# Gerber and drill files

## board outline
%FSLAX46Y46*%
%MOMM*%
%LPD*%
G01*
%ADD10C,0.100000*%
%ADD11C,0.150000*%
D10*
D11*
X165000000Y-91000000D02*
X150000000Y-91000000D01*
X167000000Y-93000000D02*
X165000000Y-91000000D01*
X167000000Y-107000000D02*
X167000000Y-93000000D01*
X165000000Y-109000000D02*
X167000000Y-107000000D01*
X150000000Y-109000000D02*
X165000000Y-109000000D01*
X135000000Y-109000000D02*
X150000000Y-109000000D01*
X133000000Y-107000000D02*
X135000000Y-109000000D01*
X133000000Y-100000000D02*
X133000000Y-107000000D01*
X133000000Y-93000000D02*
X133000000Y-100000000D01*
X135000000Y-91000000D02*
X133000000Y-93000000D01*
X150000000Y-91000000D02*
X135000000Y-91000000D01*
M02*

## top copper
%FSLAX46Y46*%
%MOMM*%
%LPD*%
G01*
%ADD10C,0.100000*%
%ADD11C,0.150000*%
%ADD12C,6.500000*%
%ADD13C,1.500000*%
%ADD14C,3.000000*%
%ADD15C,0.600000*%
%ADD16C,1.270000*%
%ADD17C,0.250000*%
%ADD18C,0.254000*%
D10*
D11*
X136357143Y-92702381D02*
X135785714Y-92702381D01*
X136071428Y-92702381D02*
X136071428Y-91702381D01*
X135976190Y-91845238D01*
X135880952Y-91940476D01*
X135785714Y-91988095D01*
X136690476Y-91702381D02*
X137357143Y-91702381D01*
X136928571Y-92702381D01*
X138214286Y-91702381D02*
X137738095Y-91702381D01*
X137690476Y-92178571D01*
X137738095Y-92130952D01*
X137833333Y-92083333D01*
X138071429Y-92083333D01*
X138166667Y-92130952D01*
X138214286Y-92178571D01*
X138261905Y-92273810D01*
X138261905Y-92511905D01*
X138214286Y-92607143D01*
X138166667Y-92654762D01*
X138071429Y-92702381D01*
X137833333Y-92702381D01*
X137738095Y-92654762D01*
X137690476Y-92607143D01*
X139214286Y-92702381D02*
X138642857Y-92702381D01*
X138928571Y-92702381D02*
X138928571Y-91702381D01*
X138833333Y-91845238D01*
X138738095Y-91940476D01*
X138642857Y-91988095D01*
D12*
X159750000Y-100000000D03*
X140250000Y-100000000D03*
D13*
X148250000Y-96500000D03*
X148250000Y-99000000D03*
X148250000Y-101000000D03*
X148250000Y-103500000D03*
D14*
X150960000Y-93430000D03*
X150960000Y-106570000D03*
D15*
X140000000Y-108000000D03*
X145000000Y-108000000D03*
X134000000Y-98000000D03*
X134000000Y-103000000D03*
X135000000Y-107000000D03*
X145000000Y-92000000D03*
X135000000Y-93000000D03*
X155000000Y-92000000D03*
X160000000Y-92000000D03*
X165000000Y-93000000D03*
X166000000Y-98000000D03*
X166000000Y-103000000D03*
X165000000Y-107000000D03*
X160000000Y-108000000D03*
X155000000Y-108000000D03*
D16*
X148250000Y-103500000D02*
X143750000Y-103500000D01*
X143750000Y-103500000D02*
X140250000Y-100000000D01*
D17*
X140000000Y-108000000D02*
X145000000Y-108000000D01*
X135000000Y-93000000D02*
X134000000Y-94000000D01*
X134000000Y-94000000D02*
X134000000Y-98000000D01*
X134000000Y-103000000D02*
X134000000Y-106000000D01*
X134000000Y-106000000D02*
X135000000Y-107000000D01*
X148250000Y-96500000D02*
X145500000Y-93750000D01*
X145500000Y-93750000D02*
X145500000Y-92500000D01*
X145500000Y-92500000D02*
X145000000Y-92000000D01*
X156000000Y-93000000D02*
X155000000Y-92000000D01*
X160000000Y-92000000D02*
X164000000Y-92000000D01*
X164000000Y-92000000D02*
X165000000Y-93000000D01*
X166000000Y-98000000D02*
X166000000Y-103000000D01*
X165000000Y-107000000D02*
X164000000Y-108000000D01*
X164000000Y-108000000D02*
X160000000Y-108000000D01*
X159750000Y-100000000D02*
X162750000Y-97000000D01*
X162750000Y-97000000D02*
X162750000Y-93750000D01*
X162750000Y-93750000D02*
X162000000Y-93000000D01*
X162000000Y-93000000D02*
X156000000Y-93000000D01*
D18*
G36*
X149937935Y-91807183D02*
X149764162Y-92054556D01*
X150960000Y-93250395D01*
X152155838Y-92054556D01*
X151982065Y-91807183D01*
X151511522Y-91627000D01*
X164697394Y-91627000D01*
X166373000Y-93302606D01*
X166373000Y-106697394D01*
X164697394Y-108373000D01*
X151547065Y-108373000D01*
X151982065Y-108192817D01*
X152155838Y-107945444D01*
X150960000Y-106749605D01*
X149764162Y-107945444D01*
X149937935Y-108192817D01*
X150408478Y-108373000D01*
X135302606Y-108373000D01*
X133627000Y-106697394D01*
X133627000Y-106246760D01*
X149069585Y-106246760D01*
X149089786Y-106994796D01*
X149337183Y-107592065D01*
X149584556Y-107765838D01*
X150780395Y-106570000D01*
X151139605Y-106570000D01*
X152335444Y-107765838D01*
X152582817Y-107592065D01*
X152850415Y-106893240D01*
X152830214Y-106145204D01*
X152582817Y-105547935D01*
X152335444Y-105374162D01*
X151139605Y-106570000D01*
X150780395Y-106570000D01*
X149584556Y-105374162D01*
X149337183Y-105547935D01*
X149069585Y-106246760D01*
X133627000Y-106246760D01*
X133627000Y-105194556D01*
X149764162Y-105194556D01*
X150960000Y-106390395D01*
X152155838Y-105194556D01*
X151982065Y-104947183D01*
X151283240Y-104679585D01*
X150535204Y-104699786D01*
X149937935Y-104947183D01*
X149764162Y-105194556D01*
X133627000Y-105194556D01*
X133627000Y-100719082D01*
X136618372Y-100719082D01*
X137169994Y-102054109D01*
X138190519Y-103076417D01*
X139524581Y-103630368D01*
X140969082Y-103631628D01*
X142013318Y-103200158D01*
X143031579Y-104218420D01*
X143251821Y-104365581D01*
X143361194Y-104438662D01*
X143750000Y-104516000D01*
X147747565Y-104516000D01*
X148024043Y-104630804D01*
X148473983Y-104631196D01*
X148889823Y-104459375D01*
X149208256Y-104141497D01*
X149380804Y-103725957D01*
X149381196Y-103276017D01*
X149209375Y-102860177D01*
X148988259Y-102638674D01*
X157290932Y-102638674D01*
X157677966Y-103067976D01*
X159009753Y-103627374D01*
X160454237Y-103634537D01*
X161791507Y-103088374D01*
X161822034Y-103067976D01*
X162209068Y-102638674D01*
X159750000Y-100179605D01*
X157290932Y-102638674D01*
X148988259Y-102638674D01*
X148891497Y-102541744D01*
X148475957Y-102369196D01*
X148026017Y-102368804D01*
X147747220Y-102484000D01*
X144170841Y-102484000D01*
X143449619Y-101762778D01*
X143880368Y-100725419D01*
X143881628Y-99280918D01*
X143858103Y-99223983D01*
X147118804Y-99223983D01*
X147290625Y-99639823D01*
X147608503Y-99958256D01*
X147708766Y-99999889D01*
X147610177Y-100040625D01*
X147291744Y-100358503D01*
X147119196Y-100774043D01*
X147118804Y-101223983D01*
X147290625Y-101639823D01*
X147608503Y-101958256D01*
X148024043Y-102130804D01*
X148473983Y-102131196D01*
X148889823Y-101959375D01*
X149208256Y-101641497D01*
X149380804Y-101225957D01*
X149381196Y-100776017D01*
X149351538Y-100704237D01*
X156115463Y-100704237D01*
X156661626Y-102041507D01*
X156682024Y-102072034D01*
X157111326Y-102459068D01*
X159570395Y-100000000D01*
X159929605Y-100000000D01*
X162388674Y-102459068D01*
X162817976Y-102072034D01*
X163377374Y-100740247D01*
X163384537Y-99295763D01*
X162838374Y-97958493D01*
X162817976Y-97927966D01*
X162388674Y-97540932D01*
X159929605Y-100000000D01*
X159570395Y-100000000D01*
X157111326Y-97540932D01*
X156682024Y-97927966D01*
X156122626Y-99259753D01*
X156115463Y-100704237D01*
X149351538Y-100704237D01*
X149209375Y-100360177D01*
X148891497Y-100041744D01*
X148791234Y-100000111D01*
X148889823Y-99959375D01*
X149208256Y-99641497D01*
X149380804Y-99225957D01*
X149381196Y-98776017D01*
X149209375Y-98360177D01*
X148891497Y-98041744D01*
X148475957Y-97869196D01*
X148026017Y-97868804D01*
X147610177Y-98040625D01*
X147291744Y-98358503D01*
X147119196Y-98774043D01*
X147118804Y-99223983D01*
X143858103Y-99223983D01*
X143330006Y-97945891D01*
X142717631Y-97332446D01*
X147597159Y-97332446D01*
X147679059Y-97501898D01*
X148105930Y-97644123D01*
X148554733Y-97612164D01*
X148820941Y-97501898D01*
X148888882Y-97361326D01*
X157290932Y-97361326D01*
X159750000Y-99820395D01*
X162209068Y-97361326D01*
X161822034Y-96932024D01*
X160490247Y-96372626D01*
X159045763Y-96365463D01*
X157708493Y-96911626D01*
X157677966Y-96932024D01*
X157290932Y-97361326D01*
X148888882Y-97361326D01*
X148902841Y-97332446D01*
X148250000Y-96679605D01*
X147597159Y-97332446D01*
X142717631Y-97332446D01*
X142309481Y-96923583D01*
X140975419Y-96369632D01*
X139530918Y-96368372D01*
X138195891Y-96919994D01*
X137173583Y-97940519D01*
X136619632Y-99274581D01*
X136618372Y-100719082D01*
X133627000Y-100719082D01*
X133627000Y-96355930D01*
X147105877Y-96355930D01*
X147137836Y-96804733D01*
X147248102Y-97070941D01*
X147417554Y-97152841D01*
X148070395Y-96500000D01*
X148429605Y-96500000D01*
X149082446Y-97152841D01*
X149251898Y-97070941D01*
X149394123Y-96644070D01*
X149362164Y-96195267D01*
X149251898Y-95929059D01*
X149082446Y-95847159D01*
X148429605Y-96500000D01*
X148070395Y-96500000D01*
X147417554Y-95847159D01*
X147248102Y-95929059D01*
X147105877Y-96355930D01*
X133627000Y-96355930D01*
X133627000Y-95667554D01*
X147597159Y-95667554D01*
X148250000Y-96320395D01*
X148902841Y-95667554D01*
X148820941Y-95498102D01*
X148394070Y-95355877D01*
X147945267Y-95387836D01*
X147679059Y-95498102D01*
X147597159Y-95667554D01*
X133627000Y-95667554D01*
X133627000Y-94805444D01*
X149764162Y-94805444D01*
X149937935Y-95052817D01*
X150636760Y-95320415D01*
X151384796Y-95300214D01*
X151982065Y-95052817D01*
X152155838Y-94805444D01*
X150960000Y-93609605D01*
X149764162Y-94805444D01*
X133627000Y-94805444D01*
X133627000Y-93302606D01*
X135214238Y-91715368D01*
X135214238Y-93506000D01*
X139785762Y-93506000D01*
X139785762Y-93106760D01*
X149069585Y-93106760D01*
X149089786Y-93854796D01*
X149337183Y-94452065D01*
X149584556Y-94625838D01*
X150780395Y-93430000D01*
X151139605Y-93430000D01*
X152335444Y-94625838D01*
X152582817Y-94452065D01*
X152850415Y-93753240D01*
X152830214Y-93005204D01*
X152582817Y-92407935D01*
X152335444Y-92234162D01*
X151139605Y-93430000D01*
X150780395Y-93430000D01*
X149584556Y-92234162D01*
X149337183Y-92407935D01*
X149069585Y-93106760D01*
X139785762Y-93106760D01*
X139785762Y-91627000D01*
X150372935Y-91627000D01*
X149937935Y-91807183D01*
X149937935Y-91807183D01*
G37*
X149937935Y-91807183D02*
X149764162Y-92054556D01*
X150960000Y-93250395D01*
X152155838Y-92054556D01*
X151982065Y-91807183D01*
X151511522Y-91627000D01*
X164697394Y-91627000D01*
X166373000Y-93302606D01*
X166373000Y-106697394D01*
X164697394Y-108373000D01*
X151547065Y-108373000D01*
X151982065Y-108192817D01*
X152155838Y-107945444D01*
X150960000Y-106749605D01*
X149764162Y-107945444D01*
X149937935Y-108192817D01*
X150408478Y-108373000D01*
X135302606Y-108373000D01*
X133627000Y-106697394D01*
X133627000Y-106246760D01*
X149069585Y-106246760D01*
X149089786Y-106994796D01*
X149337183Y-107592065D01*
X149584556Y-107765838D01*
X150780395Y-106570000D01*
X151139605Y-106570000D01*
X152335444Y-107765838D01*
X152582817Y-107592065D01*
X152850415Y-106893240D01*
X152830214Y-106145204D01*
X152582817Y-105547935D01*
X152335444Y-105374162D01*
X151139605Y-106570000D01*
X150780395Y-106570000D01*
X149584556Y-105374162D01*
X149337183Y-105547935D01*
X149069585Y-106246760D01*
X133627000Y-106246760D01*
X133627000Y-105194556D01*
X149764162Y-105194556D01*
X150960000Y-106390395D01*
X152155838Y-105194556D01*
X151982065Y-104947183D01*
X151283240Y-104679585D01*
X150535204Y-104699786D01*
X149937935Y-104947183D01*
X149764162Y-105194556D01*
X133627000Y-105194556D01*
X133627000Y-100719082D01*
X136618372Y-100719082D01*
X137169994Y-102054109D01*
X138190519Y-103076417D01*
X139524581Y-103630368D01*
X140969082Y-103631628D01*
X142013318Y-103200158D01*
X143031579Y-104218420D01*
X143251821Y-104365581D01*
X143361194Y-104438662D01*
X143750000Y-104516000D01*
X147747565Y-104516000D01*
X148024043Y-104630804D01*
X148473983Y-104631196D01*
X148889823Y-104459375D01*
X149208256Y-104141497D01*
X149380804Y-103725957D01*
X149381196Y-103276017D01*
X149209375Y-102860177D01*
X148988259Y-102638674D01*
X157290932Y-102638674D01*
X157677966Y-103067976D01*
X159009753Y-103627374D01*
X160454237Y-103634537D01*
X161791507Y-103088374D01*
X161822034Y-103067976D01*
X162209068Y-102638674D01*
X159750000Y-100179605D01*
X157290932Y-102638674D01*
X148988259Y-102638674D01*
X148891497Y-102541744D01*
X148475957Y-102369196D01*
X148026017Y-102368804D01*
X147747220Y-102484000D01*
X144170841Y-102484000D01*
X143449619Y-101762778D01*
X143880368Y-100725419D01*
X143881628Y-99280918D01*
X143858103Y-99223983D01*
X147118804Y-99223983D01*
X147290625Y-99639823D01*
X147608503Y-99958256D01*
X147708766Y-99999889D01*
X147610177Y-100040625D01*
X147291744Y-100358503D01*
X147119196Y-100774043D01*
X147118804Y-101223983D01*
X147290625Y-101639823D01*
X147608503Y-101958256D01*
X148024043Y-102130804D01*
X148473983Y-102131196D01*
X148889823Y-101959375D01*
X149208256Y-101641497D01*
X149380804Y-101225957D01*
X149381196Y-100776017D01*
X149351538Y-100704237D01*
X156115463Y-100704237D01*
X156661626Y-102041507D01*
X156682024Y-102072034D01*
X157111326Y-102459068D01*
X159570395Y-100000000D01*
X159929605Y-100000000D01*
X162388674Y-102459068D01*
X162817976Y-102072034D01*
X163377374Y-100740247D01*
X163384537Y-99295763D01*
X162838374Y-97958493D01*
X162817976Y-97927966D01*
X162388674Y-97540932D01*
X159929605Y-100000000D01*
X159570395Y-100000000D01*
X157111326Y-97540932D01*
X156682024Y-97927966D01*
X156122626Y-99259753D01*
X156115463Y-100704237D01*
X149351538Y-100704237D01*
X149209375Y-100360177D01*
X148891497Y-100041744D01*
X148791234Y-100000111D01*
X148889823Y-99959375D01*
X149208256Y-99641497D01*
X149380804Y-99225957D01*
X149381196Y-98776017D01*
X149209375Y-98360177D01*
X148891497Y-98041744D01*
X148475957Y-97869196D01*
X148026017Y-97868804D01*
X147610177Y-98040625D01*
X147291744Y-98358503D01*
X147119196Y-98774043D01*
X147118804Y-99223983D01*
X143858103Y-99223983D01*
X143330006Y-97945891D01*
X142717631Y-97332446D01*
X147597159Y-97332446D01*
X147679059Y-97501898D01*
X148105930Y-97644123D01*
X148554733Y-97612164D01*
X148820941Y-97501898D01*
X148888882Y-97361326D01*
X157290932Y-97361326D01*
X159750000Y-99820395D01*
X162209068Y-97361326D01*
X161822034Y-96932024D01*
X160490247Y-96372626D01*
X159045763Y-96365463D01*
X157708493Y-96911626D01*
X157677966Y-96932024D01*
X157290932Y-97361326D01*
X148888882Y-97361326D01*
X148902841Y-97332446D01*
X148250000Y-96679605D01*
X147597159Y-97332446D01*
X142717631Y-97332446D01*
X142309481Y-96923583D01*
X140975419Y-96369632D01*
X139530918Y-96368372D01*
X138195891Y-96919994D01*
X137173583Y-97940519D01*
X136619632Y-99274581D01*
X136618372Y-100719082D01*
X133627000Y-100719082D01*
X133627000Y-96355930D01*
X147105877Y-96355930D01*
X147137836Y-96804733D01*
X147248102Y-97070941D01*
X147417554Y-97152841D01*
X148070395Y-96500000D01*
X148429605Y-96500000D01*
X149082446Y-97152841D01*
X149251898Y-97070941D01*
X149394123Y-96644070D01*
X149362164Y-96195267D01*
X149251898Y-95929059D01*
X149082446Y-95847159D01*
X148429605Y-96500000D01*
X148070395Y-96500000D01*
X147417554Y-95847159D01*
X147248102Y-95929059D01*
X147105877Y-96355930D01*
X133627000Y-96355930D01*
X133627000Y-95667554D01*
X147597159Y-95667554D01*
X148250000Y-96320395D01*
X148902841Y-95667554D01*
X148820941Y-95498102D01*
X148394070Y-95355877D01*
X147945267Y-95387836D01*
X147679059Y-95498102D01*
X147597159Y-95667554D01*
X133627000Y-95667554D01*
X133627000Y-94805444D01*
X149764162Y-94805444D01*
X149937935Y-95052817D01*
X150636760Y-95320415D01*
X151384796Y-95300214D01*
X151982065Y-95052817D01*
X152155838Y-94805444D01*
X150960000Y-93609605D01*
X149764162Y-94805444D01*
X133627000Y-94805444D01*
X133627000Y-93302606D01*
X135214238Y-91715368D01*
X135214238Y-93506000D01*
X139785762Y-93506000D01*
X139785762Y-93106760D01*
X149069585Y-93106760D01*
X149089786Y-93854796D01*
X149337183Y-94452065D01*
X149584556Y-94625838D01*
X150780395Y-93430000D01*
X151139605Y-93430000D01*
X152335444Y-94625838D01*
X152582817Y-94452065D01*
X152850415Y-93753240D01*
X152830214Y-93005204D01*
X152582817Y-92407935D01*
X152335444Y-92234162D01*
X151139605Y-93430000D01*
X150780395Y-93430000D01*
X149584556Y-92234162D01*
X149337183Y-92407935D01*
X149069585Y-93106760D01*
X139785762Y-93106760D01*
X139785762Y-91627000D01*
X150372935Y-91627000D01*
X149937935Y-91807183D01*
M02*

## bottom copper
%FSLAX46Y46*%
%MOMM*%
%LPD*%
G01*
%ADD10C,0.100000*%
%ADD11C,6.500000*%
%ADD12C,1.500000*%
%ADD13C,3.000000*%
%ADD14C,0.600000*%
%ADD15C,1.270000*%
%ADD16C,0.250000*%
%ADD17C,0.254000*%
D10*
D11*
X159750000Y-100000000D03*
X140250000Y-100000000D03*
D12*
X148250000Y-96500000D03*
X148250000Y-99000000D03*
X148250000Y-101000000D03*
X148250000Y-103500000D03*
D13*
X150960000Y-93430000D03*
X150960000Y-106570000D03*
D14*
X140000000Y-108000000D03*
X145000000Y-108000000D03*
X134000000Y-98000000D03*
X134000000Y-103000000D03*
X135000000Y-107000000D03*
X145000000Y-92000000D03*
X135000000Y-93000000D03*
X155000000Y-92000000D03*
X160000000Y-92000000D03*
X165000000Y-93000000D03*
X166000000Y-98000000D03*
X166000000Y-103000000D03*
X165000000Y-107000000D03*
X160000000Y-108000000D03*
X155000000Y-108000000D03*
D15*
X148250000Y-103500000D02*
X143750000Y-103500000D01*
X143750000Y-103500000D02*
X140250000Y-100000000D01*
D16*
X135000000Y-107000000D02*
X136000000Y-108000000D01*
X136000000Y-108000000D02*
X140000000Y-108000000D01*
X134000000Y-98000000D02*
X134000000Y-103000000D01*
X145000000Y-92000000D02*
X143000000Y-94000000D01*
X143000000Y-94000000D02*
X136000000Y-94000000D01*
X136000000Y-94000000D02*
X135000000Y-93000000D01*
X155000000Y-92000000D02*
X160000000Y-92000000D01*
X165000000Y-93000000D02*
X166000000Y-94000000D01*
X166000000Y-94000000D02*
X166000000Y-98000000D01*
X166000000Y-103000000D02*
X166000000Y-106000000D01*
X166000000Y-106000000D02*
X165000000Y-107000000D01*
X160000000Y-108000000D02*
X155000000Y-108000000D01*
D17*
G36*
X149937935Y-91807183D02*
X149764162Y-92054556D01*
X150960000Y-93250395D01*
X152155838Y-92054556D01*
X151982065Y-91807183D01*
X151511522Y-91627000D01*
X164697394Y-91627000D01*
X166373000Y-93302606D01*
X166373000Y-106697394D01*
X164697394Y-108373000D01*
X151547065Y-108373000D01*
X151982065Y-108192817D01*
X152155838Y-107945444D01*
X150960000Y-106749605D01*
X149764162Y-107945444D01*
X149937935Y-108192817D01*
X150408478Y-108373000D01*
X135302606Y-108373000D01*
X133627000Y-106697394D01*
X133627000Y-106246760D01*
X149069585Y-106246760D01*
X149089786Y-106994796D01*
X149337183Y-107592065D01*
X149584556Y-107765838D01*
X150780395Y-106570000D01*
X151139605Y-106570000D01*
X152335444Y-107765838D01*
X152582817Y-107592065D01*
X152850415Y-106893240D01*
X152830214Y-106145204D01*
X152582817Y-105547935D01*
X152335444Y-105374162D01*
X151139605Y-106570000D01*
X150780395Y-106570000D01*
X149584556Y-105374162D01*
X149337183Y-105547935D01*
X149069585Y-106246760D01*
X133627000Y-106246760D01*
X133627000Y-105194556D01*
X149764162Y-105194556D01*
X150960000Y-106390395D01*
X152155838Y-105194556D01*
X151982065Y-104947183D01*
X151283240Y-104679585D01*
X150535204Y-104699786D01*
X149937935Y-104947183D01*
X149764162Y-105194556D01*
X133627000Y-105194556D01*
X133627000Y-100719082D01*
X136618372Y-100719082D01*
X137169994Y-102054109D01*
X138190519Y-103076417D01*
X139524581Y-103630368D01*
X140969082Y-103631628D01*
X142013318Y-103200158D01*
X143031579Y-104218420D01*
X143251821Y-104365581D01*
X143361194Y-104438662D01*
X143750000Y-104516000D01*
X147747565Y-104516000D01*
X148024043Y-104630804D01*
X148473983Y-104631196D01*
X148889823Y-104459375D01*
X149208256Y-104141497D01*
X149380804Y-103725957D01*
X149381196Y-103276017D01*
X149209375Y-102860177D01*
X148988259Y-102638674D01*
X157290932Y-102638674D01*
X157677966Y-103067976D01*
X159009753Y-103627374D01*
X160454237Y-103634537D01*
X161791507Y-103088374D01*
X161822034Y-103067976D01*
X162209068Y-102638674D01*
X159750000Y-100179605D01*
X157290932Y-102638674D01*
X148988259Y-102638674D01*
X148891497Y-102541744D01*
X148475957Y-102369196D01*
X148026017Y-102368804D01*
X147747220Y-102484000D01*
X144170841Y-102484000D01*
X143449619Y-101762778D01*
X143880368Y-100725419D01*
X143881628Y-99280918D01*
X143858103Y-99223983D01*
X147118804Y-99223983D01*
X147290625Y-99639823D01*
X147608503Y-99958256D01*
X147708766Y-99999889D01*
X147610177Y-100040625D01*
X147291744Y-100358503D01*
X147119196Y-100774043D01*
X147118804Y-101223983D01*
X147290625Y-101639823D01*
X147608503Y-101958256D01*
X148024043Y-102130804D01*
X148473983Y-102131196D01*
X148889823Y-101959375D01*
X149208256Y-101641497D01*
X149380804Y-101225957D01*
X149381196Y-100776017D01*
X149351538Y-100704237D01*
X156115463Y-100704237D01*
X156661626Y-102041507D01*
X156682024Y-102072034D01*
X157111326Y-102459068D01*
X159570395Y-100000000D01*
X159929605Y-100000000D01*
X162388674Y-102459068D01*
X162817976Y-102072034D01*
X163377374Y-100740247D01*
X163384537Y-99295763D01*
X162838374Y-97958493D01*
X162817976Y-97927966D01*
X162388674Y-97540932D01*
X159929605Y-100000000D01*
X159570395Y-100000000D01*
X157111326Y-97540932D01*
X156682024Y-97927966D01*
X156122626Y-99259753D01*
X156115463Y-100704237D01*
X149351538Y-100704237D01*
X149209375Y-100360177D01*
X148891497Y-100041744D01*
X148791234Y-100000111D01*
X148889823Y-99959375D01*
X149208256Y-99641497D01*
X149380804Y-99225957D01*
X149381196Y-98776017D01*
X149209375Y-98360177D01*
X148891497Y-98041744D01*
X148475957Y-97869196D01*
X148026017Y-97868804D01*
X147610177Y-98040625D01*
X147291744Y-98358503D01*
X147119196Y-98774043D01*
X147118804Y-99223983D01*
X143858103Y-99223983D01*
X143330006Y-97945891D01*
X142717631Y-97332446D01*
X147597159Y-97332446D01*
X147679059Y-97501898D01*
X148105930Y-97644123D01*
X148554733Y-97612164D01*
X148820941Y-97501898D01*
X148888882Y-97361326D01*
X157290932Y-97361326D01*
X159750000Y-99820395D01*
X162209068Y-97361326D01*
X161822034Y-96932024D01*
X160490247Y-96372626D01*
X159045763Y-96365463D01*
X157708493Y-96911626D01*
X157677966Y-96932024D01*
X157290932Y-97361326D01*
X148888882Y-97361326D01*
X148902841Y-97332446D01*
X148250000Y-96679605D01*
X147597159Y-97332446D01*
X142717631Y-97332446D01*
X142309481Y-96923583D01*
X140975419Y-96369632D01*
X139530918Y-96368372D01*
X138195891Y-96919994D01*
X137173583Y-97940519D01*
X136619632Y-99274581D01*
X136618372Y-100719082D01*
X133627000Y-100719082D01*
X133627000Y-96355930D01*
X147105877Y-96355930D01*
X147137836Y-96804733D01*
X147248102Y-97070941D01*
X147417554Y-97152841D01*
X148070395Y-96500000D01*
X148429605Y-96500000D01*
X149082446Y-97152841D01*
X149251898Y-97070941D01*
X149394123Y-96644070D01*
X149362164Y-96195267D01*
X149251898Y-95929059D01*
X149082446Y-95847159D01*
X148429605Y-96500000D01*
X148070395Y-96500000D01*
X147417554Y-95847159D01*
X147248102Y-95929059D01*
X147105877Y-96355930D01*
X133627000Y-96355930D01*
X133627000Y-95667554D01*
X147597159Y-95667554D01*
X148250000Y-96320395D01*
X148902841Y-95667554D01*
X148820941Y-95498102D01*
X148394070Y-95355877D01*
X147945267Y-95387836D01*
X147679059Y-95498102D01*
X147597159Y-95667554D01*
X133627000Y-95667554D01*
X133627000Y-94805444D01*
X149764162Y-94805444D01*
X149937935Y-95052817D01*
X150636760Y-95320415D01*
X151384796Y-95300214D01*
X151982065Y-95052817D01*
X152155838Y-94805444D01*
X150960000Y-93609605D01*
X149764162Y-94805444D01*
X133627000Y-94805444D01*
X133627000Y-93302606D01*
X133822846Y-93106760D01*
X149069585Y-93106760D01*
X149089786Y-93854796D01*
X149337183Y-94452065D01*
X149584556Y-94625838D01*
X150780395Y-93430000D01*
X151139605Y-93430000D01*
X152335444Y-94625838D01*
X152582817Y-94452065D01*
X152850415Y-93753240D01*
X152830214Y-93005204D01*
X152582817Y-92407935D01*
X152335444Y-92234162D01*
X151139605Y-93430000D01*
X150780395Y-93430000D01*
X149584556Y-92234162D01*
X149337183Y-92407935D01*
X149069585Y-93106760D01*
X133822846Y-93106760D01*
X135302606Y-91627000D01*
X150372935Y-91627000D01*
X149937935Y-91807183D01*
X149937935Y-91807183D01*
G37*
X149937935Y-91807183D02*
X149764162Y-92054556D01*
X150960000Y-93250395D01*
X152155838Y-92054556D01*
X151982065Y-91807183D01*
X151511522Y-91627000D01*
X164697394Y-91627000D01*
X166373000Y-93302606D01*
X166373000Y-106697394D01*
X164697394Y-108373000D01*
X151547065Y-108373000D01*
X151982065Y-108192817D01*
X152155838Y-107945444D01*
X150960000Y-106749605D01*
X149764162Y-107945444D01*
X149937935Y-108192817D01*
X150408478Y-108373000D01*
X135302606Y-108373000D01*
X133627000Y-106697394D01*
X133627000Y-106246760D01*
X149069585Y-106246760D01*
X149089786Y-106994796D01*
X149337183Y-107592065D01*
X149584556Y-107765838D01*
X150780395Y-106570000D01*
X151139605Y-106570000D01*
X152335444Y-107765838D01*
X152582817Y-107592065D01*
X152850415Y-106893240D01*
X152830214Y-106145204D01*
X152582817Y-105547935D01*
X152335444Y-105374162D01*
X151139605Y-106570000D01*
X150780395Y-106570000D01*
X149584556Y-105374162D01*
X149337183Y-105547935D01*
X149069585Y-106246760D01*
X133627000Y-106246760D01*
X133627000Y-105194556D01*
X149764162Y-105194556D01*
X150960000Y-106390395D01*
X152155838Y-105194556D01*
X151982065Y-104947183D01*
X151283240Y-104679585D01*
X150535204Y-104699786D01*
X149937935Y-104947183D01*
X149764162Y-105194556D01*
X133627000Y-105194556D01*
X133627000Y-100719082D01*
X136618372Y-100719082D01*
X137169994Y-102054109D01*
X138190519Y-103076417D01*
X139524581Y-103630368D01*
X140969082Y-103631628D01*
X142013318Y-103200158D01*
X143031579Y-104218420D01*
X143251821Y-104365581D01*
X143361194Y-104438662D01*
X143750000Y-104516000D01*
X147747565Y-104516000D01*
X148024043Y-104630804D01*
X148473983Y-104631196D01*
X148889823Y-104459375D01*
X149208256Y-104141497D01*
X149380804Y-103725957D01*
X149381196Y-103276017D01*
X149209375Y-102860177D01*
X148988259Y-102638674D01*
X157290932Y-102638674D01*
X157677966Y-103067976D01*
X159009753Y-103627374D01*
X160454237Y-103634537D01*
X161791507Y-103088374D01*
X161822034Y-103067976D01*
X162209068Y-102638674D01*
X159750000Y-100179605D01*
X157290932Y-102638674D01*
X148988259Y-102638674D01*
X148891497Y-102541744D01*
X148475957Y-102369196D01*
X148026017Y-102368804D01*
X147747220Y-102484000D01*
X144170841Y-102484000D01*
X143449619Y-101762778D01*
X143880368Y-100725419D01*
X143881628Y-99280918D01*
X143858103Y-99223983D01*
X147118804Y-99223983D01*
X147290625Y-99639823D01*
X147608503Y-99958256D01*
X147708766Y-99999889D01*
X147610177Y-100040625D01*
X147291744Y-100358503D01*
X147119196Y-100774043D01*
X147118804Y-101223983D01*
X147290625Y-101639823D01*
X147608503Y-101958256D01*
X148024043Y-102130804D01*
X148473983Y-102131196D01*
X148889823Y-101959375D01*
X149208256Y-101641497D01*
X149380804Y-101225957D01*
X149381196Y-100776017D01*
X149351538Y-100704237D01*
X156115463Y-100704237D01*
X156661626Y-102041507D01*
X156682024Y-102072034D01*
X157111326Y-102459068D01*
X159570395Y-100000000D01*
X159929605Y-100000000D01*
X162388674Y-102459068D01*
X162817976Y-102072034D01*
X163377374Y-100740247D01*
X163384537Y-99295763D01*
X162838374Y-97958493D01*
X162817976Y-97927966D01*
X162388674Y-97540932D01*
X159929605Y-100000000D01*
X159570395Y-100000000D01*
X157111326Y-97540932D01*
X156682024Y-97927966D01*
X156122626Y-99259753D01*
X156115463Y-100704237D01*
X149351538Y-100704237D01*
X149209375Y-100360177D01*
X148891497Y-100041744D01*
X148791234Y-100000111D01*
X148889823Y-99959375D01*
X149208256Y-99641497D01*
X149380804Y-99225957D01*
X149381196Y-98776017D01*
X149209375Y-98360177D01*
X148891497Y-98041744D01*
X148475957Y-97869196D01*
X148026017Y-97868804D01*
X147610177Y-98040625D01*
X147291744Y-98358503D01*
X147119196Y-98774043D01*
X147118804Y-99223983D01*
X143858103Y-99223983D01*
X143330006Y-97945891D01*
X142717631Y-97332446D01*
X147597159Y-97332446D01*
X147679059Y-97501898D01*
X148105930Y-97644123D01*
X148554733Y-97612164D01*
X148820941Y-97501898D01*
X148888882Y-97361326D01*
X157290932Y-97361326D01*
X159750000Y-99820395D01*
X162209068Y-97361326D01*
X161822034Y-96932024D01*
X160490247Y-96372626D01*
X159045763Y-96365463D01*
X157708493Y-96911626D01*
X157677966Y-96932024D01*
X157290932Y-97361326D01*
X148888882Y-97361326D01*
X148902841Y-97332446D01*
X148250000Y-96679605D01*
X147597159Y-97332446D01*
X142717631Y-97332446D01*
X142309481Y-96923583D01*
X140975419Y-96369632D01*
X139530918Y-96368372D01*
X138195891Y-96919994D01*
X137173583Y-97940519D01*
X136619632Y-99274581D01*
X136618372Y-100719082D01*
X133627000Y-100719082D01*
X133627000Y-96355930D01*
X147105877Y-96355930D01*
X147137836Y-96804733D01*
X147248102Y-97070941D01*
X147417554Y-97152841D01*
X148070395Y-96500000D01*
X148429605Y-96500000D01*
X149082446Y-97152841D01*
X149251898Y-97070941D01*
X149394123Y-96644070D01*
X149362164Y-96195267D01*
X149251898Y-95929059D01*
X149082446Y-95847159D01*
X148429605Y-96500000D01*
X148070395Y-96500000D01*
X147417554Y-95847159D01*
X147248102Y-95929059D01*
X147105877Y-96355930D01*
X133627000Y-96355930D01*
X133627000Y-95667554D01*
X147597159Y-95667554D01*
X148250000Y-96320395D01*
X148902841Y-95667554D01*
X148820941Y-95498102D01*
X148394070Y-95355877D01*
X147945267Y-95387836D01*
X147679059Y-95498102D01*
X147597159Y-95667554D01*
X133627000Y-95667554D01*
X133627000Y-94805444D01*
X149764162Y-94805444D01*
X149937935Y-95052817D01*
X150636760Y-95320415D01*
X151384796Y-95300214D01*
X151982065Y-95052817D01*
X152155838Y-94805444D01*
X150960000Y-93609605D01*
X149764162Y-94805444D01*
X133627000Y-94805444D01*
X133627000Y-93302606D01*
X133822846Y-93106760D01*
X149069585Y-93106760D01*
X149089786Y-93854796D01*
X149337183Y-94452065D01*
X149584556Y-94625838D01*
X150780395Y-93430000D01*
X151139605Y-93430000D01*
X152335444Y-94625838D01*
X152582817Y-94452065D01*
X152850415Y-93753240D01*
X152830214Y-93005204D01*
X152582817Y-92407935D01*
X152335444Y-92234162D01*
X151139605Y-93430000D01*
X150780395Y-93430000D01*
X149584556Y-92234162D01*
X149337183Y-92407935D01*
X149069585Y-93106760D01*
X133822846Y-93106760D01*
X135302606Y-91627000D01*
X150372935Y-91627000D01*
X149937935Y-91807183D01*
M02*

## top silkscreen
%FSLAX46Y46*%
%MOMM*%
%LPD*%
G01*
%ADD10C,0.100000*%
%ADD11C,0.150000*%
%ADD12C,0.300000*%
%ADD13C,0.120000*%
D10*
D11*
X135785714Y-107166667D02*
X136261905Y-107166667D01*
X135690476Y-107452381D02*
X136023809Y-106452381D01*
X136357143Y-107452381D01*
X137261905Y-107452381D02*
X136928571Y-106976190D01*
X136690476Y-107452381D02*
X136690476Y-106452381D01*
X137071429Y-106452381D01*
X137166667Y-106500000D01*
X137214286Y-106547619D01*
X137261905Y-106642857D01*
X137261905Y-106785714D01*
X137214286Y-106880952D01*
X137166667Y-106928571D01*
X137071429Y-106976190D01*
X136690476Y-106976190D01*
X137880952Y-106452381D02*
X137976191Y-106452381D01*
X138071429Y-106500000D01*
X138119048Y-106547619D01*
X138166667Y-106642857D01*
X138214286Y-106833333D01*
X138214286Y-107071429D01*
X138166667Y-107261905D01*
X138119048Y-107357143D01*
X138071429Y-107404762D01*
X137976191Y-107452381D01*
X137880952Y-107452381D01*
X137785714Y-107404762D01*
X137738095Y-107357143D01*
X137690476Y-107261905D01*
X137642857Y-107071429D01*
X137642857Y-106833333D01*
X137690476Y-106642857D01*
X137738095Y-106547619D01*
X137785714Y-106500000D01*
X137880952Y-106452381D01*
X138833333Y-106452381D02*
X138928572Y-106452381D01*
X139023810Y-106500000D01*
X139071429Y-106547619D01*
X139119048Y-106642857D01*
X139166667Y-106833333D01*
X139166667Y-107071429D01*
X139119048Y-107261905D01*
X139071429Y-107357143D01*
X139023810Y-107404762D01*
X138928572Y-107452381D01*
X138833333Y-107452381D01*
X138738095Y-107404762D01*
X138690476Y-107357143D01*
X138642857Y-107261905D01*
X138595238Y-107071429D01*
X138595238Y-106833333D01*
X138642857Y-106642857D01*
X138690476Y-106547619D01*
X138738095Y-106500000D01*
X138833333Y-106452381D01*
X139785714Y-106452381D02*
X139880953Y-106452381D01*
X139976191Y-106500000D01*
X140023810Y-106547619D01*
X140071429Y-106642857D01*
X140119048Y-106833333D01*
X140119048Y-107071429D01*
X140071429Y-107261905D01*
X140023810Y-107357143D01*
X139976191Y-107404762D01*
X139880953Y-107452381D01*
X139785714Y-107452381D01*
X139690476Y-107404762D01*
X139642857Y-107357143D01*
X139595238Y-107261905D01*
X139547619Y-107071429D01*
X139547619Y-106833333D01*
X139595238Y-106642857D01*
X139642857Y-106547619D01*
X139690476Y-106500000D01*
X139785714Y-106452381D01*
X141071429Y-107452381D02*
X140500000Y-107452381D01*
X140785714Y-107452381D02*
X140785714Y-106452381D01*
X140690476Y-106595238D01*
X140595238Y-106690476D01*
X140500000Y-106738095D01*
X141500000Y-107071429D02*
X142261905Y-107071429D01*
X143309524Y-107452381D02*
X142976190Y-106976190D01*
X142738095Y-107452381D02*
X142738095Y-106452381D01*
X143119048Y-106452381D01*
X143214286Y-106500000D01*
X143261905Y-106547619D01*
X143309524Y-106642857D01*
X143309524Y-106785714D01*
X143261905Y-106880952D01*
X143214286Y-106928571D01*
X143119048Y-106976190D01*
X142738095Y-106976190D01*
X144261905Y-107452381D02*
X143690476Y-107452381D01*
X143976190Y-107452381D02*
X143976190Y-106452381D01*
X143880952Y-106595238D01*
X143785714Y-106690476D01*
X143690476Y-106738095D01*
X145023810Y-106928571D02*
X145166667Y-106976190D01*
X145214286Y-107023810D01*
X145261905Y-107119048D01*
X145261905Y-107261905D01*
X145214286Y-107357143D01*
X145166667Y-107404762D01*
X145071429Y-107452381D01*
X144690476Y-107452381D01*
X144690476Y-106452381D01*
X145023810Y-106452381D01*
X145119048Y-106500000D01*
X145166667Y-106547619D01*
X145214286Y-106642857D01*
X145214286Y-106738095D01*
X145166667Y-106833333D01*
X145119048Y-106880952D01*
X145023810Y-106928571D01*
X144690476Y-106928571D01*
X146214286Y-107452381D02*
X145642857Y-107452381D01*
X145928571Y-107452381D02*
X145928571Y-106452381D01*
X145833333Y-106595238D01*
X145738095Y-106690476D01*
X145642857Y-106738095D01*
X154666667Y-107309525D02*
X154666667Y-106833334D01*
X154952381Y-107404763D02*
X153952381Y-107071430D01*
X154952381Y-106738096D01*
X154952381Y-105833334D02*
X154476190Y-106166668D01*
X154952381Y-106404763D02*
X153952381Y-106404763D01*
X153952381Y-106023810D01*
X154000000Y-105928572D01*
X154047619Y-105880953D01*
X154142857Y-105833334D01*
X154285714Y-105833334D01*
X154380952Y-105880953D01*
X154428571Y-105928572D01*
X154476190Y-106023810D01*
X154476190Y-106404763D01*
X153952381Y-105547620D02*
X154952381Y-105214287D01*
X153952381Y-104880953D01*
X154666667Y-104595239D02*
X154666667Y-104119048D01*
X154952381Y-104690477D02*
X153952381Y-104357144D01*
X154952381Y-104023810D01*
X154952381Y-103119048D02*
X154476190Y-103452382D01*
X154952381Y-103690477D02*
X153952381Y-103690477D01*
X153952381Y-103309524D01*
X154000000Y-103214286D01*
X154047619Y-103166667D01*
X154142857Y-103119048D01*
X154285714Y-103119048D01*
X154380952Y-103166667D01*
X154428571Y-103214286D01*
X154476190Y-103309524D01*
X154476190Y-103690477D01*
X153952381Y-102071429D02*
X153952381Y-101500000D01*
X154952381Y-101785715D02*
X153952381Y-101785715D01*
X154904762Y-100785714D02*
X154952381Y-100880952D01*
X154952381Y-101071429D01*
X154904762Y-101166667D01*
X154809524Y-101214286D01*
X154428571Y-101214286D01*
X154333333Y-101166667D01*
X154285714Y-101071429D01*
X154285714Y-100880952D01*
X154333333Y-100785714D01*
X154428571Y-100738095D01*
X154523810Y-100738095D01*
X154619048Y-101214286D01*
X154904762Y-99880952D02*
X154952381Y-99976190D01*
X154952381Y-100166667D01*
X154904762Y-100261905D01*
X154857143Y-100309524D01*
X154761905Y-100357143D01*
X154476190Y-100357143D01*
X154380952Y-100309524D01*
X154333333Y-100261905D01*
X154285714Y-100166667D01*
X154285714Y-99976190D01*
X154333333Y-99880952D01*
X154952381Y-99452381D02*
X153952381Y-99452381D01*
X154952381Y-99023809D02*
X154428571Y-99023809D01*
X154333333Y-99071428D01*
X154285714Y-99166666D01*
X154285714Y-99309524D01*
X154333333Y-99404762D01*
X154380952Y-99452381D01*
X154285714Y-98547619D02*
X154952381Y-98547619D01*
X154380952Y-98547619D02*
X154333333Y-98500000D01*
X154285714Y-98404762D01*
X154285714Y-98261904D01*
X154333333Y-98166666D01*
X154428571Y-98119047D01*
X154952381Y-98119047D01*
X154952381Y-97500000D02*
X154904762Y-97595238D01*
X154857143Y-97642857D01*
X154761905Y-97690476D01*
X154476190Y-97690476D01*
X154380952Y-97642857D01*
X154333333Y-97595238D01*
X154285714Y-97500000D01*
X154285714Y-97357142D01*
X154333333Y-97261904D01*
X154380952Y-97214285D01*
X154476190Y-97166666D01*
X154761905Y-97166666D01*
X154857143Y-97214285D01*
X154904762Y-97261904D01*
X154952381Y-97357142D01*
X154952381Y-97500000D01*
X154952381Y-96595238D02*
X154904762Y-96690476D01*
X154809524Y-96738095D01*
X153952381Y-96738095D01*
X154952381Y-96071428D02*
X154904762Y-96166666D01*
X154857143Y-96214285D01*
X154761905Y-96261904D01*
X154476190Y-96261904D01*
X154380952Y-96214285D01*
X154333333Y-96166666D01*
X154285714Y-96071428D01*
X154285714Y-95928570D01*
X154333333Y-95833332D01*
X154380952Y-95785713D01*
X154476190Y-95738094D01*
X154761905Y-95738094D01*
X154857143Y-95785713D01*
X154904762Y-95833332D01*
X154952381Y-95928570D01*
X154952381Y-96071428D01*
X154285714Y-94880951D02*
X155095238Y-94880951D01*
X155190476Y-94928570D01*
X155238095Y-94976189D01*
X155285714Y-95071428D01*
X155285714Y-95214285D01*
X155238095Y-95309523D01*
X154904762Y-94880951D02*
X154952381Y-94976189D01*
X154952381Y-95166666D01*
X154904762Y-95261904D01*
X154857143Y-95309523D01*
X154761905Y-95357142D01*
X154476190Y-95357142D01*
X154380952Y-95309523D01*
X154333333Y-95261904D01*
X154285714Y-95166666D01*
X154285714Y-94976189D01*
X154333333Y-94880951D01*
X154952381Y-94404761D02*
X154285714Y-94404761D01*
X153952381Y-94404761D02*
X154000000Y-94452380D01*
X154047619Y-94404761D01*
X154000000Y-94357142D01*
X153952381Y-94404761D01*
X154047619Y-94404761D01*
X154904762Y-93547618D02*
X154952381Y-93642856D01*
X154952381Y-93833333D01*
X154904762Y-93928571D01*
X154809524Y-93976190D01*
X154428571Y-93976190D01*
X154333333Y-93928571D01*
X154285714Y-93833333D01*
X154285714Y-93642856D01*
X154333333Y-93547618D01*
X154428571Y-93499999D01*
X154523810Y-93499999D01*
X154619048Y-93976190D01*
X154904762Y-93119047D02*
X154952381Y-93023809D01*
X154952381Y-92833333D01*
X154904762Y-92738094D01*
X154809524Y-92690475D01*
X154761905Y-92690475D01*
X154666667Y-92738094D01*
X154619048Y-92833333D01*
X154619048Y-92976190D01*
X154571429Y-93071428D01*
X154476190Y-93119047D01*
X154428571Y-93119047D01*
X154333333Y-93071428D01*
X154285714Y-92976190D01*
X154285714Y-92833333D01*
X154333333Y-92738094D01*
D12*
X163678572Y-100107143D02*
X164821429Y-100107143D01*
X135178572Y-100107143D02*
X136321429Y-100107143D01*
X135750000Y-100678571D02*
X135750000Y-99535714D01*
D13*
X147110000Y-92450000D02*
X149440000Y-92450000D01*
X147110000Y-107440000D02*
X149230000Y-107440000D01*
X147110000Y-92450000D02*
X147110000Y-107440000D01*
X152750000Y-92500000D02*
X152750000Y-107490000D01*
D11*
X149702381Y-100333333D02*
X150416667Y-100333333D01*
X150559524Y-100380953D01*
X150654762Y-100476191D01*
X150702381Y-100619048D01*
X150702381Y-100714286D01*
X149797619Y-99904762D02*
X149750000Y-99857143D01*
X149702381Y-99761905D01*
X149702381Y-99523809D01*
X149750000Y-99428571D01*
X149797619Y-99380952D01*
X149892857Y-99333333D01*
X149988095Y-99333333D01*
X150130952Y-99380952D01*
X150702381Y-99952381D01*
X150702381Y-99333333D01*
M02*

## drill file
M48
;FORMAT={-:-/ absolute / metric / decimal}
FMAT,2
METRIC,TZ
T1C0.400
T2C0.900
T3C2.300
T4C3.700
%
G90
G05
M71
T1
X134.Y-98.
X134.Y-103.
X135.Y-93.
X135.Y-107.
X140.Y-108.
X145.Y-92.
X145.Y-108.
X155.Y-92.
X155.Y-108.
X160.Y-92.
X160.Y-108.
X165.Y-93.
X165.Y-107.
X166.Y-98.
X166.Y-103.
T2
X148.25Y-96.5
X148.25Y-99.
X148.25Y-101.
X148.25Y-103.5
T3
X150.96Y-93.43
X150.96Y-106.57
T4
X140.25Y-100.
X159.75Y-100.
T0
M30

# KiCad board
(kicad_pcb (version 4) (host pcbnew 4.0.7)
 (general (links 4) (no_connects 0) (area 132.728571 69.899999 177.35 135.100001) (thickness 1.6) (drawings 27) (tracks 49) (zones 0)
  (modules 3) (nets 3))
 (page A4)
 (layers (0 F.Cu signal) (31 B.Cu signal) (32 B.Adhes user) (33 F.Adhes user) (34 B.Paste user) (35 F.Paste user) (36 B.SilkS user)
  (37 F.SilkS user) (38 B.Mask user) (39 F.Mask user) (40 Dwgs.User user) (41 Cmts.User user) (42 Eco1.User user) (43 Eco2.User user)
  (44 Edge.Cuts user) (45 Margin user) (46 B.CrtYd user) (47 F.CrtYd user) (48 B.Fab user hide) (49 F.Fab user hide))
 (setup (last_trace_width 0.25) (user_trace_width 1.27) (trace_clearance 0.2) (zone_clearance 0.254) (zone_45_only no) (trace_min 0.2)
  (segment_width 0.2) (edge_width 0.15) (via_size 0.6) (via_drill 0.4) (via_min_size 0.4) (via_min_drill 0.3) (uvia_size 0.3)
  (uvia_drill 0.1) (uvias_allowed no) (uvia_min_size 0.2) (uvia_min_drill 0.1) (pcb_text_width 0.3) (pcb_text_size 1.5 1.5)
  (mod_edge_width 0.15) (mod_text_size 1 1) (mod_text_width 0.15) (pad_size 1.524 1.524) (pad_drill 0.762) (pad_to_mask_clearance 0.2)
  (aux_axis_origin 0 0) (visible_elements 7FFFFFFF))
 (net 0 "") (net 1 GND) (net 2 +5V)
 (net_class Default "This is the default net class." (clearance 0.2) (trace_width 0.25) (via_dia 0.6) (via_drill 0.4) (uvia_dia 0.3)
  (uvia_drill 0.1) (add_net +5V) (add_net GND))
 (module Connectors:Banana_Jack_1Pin (layer F.Cu) (at 159.75 100)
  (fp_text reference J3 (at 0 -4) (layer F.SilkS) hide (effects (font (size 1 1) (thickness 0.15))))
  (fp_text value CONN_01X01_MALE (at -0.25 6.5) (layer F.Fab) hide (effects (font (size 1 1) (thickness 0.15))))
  (pad 1 thru_hole circle (at 0 0) (size 6.5 6.5) (drill 3.7) (layers *.Cu *.Mask) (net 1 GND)))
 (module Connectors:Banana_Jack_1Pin (layer F.Cu) (at 140.25 100)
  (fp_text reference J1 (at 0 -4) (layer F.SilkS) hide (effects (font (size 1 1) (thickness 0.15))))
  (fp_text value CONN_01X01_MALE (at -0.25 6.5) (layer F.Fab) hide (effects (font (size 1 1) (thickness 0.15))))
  (pad 1 thru_hole circle (at 0 0) (size 6.5 6.5) (drill 3.7) (layers *.Cu *.Mask) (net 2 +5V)))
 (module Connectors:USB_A (layer F.Cu) (at 148.25 103.5 90)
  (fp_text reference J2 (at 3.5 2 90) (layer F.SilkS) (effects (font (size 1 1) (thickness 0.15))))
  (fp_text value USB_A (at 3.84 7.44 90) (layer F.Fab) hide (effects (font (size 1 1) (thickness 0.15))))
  (fp_line (start 11.05 -1.14) (end 11.05 1.19) (layer F.SilkS) (width 0.12))
  (fp_line (start -3.94 -1.14) (end -3.94 0.98) (layer F.SilkS) (width 0.12))
  (fp_line (start 11.05 -1.14) (end -3.94 -1.14) (layer F.SilkS) (width 0.12))
  (fp_line (start 11 4.5) (end -3.99 4.5) (layer F.SilkS) (width 0.12))
  (pad 4 thru_hole circle (at 7 0) (size 1.5 1.5) (drill 0.9) (layers *.Cu *.Mask) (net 1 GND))
  (pad 3 thru_hole circle (at 4.5 0) (size 1.5 1.5) (drill 0.9) (layers *.Cu *.Mask))
  (pad 2 thru_hole circle (at 2.5 0) (size 1.5 1.5) (drill 0.9) (layers *.Cu *.Mask))
  (pad 1 thru_hole circle (at 0 0) (size 1.5 1.5) (drill 0.9) (layers *.Cu *.Mask) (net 2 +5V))
  (pad 5 thru_hole circle (at 10.07 2.71) (size 3 3) (drill 2.3) (layers *.Cu *.Mask) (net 1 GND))
  (pad 5 thru_hole circle (at -3.07 2.71) (size 3 3) (drill 2.3) (layers *.Cu *.Mask) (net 1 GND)))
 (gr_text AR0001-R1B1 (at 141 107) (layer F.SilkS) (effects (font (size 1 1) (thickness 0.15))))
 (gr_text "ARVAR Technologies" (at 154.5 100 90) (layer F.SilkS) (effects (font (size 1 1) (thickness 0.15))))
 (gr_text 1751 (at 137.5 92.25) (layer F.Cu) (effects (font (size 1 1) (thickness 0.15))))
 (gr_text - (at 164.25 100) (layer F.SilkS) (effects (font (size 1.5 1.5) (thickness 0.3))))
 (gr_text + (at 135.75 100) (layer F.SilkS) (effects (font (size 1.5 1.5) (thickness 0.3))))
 (gr_line (start 165 91) (end 150 91) (layer Edge.Cuts) (width 0.15))
 (gr_line (start 167 93) (end 165 91) (layer Edge.Cuts) (width 0.15))
 (gr_line (start 167 107) (end 167 93) (layer Edge.Cuts) (width 0.15))
 (gr_line (start 165 109) (end 167 107) (layer Edge.Cuts) (width 0.15))
 (gr_line (start 150 109) (end 165 109) (layer Edge.Cuts) (width 0.15))
 (gr_line (start 135 109) (end 150 109) (layer Edge.Cuts) (width 0.15))
 (gr_line (start 133 107) (end 135 109) (layer Edge.Cuts) (width 0.15))
 (gr_line (start 133 100) (end 133 107) (layer Edge.Cuts) (width 0.15))
 (gr_line (start 133 93) (end 133 100) (layer Edge.Cuts) (width 0.15))
 (gr_line (start 135 91) (end 133 93) (layer Edge.Cuts) (width 0.15))
 (gr_line (start 150 91) (end 135 91) (layer Edge.Cuts) (width 0.15))
 (segment (start 148.25 103.5) (end 143.75 103.5) (width 1.27) (layer B.Cu) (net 2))
 (segment (start 143.75 103.5) (end 140.25 100) (width 1.27) (layer B.Cu) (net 2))
 (segment (start 148.25 103.5) (end 143.75 103.5) (width 1.27) (layer F.Cu) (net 2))
 (segment (start 143.75 103.5) (end 140.25 100) (width 1.27) (layer F.Cu) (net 2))
 (segment (start 135 107) (end 136 108) (width 0.25) (layer B.Cu) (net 1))
 (segment (start 136 108) (end 140 108) (width 0.25) (layer B.Cu) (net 1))
 (via (at 140 108) (size 0.6) (drill 0.4) (layers F.Cu B.Cu) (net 1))
 (segment (start 140 108) (end 145 108) (width 0.25) (layer F.Cu) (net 1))
 (via (at 145 108) (size 0.6) (drill 0.4) (layers F.Cu B.Cu) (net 1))
 (segment (start 135 93) (end 134 94) (width 0.25) (layer F.Cu) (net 1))
 (segment (start 134 94) (end 134 98) (width 0.25) (layer F.Cu) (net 1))
 (via (at 134 98) (size 0.6) (drill 0.4) (layers F.Cu B.Cu) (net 1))
 (segment (start 134 98) (end 134 103) (width 0.25) (layer B.Cu) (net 1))
 (via (at 134 103) (size 0.6) (drill 0.4) (layers F.Cu B.Cu) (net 1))
 (segment (start 134 103) (end 134 106) (width 0.25) (layer F.Cu) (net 1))
 (segment (start 134 106) (end 135 107) (width 0.25) (layer F.Cu) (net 1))
 (via (at 135 107) (size 0.6) (drill 0.4) (layers F.Cu B.Cu) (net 1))
 (segment (start 148.25 96.5) (end 145.5 93.75) (width 0.25) (layer F.Cu) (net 1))
 (segment (start 145.5 93.75) (end 145.5 92.5) (width 0.25) (layer F.Cu) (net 1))
 (segment (start 145.5 92.5) (end 145 92) (width 0.25) (layer F.Cu) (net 1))
 (via (at 145 92) (size 0.6) (drill 0.4) (layers F.Cu B.Cu) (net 1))
 (segment (start 145 92) (end 143 94) (width 0.25) (layer B.Cu) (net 1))
 (segment (start 143 94) (end 136 94) (width 0.25) (layer B.Cu) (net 1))
 (segment (start 136 94) (end 135 93) (width 0.25) (layer B.Cu) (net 1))
 (via (at 135 93) (size 0.6) (drill 0.4) (layers F.Cu B.Cu) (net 1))
 (segment (start 156 93) (end 155 92) (width 0.25) (layer F.Cu) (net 1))
 (via (at 155 92) (size 0.6) (drill 0.4) (layers F.Cu B.Cu) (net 1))
 (segment (start 155 92) (end 160 92) (width 0.25) (layer B.Cu) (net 1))
 (via (at 160 92) (size 0.6) (drill 0.4) (layers F.Cu B.Cu) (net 1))
 (segment (start 160 92) (end 164 92) (width 0.25) (layer F.Cu) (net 1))
 (segment (start 164 92) (end 165 93) (width 0.25) (layer F.Cu) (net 1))
 (via (at 165 93) (size 0.6) (drill 0.4) (layers F.Cu B.Cu) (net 1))
 (segment (start 165 93) (end 166 94) (width 0.25) (layer B.Cu) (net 1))
 (segment (start 166 94) (end 166 98) (width 0.25) (layer B.Cu) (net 1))
 (via (at 166 98) (size 0.6) (drill 0.4) (layers F.Cu B.Cu) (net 1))
 (segment (start 166 98) (end 166 103) (width 0.25) (layer F.Cu) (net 1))
 (via (at 166 103) (size 0.6) (drill 0.4) (layers F.Cu B.Cu) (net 1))
 (segment (start 166 103) (end 166 106) (width 0.25) (layer B.Cu) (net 1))
 (segment (start 166 106) (end 165 107) (width 0.25) (layer B.Cu) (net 1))
 (via (at 165 107) (size 0.6) (drill 0.4) (layers F.Cu B.Cu) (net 1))
 (segment (start 165 107) (end 164 108) (width 0.25) (layer F.Cu) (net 1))
 (segment (start 164 108) (end 160 108) (width 0.25) (layer F.Cu) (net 1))
 (via (at 160 108) (size 0.6) (drill 0.4) (layers F.Cu B.Cu) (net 1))
 (segment (start 160 108) (end 155 108) (width 0.25) (layer B.Cu) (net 1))
 (via (at 155 108) (size 0.6) (drill 0.4) (layers F.Cu B.Cu) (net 1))
 (segment (start 159.75 100) (end 162.75 97) (width 0.25) (layer F.Cu) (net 1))
 (segment (start 162.75 97) (end 162.75 93.75) (width 0.25) (layer F.Cu) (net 1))
 (segment (start 162.75 93.75) (end 162 93) (width 0.25) (layer F.Cu) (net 1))
 (segment (start 162 93) (end 156 93) (width 0.25) (layer F.Cu) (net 1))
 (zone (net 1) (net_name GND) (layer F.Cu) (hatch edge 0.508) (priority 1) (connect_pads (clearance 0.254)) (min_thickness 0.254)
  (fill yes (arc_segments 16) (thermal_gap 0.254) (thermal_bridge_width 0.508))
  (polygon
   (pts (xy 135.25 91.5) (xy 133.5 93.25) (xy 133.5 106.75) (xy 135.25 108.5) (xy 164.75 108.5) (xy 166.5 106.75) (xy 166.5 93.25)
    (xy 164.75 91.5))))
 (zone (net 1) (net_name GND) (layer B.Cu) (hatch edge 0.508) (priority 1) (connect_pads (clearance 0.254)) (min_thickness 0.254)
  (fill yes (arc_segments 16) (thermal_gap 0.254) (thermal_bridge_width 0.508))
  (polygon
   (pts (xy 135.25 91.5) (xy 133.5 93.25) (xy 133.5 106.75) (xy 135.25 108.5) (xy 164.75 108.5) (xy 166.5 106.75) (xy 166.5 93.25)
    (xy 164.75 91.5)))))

